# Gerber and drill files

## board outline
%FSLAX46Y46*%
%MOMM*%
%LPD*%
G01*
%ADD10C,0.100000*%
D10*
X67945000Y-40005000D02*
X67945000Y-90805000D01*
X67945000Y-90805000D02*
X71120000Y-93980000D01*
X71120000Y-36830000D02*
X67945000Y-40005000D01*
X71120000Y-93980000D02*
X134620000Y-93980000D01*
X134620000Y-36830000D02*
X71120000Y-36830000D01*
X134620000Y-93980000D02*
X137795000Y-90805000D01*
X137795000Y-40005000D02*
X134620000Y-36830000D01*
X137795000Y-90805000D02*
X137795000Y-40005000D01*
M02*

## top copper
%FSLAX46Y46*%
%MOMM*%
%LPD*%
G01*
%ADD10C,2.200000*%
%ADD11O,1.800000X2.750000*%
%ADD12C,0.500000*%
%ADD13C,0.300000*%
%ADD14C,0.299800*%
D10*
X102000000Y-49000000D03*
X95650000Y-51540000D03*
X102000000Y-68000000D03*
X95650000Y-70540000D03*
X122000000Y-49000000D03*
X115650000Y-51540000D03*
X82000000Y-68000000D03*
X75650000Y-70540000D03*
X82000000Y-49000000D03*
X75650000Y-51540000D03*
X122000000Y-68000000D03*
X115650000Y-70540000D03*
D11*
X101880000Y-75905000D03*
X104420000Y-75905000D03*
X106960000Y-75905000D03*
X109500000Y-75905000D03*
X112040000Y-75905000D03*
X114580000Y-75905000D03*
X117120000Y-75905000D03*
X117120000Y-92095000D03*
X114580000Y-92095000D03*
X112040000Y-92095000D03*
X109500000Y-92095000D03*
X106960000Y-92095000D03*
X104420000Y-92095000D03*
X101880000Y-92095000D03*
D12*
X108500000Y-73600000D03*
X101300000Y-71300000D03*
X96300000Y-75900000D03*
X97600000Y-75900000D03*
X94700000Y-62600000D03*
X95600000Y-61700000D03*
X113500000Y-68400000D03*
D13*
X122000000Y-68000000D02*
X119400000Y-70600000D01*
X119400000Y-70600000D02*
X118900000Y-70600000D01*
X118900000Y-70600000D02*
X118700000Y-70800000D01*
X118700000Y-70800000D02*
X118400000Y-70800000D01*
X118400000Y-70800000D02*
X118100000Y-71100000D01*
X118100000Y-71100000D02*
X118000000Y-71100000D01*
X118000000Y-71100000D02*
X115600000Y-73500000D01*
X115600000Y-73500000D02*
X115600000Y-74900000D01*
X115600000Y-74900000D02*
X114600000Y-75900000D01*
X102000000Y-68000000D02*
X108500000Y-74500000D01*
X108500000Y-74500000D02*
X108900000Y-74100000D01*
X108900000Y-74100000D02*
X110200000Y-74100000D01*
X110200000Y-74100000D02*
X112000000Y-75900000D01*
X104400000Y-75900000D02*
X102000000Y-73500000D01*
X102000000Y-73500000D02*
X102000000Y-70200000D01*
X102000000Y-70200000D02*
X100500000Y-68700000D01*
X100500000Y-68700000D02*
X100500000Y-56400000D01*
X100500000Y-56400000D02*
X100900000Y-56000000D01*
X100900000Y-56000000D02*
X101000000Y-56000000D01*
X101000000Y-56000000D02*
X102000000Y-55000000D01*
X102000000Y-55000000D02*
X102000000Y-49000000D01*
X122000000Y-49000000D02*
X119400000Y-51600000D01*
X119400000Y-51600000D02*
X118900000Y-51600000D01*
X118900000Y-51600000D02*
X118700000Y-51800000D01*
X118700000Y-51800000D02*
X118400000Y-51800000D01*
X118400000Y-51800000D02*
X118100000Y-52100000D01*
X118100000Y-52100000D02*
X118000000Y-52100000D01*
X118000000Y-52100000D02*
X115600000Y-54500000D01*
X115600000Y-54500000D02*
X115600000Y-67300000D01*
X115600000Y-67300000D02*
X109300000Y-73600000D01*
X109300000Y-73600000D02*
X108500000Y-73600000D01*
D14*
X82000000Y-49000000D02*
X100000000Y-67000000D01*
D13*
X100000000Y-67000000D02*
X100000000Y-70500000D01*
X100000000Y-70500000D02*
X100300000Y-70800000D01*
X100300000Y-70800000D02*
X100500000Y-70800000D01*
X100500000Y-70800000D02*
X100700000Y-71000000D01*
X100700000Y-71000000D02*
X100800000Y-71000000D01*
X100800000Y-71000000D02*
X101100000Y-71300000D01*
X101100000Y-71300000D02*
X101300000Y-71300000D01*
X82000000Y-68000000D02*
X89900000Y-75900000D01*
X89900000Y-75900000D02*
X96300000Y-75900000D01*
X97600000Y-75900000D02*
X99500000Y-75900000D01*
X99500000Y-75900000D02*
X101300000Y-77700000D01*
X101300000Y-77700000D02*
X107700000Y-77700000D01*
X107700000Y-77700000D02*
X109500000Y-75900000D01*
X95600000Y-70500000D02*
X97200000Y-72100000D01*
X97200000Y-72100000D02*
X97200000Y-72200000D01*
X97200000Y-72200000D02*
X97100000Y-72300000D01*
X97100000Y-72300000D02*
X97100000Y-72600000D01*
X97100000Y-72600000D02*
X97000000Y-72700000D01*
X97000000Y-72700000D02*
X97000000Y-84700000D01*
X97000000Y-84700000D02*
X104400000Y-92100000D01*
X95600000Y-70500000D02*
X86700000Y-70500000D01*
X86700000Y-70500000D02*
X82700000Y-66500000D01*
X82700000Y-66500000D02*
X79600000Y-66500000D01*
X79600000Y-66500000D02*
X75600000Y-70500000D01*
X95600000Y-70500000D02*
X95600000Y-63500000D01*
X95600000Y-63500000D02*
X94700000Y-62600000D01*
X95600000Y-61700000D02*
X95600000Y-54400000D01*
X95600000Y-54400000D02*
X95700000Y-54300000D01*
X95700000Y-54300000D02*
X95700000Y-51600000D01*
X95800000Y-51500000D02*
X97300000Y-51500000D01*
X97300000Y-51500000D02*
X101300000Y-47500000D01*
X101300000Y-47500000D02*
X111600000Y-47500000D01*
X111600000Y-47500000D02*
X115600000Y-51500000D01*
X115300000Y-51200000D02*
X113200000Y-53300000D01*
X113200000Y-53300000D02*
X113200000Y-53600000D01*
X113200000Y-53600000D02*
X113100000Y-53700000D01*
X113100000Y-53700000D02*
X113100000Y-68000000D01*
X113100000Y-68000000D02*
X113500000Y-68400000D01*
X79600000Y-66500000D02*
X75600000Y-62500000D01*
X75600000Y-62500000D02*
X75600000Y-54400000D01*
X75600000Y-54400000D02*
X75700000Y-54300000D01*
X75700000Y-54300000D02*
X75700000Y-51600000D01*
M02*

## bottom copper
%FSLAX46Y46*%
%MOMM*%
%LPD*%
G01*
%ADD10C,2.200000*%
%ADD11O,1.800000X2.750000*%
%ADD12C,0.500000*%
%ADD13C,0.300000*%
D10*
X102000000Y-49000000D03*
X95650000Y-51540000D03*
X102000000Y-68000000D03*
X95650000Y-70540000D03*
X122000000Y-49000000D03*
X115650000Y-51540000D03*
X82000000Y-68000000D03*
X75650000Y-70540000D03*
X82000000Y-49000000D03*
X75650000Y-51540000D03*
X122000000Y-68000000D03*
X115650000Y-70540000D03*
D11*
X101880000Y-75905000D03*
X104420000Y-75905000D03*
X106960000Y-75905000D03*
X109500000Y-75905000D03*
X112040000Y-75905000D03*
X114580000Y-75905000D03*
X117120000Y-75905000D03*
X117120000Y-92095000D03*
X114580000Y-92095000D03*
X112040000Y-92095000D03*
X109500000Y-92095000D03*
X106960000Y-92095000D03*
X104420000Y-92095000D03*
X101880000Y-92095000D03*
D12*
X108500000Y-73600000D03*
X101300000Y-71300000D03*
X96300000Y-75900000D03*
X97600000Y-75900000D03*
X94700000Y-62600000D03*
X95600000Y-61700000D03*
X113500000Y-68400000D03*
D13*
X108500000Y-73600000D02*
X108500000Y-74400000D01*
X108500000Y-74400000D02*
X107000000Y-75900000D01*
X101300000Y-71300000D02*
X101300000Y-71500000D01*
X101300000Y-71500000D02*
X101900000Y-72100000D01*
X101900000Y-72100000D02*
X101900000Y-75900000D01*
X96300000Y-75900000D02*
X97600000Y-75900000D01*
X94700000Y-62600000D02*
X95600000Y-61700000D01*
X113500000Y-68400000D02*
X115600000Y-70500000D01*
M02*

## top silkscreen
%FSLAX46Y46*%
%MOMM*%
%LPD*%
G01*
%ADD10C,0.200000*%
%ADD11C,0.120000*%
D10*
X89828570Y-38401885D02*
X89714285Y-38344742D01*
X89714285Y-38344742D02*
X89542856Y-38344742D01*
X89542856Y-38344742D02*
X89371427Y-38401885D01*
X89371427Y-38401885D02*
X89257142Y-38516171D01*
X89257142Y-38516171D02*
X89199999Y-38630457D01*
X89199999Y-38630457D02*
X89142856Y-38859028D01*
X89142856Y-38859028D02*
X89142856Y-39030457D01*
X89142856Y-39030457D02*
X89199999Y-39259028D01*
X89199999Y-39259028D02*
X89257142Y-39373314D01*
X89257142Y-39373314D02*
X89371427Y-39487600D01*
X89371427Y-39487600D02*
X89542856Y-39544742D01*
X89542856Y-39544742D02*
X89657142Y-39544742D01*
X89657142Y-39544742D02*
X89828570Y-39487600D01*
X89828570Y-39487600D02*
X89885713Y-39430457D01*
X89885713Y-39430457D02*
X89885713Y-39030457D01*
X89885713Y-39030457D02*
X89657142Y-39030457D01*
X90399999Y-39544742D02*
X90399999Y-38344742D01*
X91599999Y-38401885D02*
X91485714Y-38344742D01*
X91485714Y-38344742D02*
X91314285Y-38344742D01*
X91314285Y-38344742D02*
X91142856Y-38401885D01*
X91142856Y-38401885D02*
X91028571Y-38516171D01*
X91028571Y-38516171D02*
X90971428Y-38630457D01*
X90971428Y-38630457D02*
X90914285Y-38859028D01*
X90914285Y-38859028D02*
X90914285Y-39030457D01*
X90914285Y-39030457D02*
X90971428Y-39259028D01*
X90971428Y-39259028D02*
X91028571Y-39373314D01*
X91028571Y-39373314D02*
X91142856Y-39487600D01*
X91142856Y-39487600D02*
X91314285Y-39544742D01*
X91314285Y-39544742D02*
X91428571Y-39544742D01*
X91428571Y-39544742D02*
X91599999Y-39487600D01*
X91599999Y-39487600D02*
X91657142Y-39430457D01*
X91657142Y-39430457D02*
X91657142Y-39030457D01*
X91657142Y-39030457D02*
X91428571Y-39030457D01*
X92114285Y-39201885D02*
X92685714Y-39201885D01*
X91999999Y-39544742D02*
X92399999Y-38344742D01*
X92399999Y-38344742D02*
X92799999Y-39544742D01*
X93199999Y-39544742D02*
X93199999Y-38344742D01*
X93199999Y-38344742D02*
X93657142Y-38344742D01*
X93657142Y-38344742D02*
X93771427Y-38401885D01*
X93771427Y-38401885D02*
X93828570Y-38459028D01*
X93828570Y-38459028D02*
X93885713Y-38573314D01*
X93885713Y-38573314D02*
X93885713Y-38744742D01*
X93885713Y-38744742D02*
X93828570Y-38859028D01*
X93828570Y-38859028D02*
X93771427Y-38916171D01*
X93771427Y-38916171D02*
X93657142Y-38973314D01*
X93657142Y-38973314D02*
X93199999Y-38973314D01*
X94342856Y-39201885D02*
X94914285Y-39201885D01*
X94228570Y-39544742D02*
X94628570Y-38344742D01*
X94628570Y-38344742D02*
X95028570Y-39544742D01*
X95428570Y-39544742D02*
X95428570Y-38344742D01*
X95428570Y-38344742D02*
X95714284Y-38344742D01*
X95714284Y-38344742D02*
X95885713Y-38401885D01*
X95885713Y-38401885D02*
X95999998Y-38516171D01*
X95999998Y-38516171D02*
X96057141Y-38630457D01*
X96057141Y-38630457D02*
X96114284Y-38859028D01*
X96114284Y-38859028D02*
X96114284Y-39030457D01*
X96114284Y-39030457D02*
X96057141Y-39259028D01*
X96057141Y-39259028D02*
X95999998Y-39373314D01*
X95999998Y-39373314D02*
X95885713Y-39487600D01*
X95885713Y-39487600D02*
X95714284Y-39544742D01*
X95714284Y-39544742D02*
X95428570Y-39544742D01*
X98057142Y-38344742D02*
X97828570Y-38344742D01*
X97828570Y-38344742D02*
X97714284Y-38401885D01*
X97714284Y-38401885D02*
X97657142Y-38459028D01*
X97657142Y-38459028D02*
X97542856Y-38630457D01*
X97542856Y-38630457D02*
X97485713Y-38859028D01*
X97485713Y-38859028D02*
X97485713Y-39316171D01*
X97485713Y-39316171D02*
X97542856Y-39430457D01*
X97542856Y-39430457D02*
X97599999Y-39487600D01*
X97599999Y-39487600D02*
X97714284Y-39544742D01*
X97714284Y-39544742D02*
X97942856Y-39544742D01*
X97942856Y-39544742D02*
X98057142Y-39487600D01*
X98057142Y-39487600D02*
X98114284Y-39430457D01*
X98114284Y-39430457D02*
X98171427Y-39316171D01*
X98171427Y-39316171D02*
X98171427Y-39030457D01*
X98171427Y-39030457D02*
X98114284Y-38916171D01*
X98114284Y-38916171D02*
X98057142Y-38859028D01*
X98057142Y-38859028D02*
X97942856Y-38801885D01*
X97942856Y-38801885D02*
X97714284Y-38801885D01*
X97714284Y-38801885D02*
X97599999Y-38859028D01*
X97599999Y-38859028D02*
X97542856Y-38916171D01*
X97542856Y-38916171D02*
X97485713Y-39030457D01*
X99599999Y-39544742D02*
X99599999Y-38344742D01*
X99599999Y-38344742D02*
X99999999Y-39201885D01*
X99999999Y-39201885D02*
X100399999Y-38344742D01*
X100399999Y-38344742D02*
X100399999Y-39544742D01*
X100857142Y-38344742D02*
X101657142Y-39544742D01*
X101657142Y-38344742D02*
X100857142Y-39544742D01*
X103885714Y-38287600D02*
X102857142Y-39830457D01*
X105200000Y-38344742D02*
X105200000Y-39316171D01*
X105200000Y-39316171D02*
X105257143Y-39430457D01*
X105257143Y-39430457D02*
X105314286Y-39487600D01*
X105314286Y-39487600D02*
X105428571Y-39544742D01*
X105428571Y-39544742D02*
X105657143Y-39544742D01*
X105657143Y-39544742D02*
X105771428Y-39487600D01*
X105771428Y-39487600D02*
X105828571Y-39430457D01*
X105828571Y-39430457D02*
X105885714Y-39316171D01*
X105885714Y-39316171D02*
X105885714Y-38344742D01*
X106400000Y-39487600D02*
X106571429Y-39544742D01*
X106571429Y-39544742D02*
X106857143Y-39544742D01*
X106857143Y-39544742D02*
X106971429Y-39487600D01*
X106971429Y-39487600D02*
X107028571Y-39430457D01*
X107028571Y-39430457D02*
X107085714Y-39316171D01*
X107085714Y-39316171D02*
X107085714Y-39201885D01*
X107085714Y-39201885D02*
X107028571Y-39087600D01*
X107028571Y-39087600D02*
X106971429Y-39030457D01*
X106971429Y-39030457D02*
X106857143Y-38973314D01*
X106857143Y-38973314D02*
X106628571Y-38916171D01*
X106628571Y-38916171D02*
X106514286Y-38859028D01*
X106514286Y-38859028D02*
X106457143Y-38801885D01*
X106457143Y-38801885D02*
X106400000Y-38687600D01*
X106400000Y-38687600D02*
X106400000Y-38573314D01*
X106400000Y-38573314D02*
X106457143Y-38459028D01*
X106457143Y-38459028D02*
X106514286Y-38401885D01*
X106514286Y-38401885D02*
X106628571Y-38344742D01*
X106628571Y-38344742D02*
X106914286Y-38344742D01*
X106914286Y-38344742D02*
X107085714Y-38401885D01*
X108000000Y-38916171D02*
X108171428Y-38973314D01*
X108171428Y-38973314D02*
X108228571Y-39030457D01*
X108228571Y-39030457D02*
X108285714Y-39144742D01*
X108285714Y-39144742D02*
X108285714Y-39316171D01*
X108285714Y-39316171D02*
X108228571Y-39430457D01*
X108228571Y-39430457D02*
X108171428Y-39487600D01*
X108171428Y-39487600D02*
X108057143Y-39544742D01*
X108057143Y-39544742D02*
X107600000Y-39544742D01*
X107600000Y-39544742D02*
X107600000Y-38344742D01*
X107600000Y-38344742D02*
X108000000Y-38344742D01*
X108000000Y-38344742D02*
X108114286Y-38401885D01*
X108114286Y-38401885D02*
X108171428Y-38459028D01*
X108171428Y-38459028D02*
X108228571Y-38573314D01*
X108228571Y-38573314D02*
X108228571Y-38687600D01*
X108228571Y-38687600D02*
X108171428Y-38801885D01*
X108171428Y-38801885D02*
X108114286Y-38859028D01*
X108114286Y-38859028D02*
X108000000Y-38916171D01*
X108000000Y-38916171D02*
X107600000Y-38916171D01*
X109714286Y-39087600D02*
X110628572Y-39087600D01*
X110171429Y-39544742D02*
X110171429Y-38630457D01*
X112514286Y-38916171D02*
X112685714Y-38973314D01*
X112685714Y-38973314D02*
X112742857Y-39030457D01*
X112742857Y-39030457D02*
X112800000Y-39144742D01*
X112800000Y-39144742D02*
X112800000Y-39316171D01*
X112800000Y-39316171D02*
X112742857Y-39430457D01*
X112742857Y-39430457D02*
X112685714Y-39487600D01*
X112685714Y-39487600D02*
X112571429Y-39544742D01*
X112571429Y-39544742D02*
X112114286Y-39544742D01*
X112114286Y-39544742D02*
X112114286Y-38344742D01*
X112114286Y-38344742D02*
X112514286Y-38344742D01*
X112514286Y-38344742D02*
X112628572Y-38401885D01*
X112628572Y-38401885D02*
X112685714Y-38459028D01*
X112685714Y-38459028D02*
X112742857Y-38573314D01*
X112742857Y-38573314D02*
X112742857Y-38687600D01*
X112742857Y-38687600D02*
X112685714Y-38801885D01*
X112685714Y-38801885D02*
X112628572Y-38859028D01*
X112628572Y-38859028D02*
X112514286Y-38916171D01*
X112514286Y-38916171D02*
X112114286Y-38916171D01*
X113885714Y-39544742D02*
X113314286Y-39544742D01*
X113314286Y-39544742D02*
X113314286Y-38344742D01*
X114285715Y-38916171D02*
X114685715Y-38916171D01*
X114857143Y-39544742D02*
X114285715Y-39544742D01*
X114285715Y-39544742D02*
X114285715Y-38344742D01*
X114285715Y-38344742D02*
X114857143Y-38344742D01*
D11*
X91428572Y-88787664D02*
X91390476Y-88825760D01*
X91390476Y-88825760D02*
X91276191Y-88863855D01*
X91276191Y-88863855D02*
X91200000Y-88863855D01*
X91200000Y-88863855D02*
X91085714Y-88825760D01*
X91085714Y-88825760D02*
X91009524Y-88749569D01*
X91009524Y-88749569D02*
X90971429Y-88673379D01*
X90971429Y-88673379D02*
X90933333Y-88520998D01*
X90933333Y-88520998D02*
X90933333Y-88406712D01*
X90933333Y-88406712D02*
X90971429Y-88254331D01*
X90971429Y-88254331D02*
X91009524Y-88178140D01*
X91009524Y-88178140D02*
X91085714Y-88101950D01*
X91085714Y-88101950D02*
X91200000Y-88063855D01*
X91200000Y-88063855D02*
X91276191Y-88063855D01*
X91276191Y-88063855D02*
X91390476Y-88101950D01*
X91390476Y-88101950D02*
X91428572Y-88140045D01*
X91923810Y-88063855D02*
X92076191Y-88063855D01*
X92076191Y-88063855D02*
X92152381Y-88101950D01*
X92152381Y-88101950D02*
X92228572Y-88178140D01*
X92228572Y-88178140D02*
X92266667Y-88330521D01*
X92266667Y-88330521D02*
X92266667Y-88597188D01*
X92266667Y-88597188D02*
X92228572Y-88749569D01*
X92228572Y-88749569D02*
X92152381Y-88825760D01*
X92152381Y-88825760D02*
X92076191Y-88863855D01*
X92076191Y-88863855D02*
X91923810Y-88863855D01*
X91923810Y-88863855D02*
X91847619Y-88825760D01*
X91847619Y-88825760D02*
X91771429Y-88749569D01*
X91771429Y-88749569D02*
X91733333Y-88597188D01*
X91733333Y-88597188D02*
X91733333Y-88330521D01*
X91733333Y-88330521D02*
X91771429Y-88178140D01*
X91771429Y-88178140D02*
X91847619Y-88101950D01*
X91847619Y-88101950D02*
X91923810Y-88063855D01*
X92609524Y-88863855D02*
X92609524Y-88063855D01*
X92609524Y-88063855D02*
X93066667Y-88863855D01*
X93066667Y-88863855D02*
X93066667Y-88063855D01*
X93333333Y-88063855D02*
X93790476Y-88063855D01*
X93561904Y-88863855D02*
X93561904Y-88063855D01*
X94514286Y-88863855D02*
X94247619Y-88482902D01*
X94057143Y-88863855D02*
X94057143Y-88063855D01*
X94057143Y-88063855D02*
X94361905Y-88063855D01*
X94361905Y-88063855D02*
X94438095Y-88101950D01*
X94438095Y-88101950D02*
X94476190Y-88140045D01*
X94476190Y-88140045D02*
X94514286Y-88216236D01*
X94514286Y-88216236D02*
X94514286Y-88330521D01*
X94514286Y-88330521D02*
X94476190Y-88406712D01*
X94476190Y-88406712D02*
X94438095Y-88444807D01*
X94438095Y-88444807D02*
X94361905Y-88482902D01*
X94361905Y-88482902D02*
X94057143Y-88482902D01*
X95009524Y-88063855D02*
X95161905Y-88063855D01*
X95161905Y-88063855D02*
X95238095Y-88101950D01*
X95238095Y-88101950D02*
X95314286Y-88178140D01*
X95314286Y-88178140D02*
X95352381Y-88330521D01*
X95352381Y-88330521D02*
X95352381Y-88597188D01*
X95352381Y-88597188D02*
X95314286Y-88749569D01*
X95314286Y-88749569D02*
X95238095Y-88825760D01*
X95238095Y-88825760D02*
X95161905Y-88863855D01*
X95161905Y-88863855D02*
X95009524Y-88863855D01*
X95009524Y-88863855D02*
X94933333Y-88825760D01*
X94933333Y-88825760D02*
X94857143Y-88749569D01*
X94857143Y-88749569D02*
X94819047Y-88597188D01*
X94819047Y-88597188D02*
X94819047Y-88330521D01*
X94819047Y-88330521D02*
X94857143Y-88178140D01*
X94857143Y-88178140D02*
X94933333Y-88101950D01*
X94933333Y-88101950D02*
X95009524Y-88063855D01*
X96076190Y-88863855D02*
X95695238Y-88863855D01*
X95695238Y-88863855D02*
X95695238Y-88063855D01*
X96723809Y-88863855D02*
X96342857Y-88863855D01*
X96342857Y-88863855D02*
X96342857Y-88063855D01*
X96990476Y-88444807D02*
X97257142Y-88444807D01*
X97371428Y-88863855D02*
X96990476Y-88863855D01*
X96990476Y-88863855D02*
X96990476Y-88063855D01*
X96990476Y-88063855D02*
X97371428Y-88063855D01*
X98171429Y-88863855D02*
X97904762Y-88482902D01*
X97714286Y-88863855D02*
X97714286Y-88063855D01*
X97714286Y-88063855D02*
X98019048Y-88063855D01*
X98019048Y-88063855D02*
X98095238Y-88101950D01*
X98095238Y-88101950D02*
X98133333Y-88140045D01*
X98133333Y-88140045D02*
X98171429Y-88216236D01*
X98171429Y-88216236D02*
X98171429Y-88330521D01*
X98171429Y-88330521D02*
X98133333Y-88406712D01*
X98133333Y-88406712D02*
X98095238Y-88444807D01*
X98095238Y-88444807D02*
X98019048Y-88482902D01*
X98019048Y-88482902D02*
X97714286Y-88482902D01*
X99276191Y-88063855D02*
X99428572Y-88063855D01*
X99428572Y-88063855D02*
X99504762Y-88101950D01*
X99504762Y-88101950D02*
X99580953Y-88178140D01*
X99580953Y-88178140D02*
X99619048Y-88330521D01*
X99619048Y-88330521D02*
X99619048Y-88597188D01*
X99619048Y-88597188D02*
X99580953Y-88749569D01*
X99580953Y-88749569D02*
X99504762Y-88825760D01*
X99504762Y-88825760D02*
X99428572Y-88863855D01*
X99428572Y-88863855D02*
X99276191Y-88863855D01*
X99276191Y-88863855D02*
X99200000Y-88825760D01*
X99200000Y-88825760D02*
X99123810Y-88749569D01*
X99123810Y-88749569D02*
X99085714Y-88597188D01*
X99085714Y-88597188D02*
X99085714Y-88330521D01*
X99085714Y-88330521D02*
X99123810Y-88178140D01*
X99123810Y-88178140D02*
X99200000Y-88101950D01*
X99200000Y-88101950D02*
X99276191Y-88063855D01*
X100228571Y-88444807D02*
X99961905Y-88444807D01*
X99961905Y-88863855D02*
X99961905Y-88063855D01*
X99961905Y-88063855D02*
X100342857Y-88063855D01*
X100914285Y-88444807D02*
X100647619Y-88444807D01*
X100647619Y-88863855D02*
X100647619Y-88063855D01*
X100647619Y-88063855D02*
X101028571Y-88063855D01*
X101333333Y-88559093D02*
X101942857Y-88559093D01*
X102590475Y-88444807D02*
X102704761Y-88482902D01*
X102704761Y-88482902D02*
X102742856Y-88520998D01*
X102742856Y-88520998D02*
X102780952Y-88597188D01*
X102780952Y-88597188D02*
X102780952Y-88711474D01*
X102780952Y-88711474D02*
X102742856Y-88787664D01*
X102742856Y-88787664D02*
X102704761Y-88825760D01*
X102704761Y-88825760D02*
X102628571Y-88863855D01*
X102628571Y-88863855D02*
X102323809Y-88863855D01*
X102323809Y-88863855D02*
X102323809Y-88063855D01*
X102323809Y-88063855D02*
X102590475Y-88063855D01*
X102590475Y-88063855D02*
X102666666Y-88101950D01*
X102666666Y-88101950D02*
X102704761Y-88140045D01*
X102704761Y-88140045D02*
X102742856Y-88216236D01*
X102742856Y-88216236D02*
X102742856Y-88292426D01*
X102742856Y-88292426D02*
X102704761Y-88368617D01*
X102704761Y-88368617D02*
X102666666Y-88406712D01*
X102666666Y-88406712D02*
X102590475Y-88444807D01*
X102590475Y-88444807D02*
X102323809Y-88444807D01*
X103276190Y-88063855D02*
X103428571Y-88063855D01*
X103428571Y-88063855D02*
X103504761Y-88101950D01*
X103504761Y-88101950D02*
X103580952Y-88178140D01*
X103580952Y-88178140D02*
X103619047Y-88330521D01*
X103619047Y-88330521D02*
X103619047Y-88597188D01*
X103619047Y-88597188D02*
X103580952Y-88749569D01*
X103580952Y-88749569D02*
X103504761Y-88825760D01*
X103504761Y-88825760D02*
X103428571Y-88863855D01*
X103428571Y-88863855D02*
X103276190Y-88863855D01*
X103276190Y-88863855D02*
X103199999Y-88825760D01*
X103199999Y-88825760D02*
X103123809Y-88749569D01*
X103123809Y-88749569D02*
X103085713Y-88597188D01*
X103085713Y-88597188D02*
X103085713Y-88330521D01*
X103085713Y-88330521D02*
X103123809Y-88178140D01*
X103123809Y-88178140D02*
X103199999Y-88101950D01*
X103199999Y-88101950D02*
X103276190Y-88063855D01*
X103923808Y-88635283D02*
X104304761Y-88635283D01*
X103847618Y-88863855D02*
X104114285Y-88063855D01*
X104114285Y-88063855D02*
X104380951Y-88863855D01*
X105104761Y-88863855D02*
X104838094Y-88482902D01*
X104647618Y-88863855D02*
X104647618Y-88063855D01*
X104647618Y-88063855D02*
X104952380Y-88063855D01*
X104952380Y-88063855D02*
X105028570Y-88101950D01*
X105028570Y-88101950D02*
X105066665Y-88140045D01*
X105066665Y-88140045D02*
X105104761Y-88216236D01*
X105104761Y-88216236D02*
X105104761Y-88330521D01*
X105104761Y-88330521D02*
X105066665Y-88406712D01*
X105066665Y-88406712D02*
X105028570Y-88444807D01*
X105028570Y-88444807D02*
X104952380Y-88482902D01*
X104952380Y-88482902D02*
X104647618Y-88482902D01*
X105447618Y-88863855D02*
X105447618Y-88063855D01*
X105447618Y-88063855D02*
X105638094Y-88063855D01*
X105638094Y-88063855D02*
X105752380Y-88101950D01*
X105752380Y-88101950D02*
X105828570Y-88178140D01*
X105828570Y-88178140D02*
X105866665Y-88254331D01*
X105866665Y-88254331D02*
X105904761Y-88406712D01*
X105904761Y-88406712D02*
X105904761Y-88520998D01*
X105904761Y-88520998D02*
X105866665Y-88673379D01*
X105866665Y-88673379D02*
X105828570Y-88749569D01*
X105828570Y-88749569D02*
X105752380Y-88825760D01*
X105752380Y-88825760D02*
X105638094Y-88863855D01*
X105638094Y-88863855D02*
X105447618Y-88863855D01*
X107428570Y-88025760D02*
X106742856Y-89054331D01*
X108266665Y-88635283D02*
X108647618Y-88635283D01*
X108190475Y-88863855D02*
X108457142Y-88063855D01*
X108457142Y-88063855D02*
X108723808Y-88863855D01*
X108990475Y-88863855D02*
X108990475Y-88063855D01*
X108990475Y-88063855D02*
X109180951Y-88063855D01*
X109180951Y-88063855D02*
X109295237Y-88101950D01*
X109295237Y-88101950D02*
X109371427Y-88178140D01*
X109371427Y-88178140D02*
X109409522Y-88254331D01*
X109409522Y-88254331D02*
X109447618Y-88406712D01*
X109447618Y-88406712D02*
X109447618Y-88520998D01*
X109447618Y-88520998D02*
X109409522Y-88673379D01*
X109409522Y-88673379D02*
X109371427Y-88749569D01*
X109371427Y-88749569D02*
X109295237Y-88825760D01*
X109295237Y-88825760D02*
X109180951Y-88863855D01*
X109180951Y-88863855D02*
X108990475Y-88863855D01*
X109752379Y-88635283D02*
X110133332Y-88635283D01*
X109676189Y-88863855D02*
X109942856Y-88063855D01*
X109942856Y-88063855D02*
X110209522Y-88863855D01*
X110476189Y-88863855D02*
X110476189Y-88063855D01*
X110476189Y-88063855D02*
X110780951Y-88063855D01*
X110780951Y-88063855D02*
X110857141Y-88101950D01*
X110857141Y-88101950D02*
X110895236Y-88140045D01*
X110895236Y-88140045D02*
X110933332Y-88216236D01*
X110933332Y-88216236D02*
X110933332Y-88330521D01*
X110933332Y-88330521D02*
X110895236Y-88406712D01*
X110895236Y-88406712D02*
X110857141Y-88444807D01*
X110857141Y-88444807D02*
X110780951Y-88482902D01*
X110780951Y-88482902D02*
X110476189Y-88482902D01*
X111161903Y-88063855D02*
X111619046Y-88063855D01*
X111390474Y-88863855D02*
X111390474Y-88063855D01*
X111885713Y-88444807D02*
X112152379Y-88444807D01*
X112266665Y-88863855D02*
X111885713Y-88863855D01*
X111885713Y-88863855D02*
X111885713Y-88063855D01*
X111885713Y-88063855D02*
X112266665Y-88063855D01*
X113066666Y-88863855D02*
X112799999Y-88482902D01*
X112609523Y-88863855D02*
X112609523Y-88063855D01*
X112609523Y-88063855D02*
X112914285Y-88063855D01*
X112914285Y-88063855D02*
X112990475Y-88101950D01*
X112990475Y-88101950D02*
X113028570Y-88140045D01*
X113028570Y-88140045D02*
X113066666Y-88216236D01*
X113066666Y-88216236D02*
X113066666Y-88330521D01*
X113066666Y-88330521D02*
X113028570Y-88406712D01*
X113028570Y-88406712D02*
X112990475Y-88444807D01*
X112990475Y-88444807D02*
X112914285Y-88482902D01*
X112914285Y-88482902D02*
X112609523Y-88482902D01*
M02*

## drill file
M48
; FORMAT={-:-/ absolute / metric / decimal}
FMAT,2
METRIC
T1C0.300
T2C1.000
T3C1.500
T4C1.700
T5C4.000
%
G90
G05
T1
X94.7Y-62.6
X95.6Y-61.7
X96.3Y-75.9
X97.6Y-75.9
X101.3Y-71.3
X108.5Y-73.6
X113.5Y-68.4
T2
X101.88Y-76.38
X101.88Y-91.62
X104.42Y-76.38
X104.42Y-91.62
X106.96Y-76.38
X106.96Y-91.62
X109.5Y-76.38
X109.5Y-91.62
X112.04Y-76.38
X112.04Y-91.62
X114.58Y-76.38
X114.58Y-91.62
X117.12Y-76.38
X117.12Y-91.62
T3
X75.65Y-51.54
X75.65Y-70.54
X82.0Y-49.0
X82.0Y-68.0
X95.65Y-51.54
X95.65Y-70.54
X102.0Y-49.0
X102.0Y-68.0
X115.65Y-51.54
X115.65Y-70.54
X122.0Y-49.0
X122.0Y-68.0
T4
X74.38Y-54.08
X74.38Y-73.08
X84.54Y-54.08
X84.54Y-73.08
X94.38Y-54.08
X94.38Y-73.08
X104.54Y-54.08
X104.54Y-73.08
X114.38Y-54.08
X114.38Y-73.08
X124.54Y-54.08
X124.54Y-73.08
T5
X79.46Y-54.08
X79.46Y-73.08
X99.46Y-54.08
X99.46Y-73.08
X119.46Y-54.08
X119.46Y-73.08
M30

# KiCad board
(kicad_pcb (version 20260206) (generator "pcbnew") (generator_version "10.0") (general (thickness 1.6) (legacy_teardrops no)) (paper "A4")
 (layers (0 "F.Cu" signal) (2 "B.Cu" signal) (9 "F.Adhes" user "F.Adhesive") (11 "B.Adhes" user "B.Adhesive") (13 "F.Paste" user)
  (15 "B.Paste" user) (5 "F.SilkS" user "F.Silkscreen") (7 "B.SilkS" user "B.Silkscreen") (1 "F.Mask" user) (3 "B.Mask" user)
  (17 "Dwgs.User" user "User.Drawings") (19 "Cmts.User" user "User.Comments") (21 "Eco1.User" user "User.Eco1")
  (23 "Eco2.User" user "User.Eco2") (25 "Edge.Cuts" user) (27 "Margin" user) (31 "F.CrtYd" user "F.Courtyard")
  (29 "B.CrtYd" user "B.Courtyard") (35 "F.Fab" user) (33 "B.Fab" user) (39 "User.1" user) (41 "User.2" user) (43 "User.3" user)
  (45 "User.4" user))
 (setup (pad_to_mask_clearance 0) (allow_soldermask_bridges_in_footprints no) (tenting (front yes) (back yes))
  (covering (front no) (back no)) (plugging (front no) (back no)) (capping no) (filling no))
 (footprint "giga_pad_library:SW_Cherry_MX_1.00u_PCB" (layer "F.Cu") (at 102 49)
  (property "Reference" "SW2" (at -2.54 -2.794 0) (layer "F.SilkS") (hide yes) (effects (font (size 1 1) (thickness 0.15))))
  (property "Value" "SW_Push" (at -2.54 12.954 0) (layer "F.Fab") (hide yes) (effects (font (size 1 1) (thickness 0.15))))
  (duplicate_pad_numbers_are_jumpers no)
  (pad "" np_thru_hole circle (at -7.62 5.08) (size 1.7 1.7) (drill 1.7) (layers "*.Cu" "*.Mask"))
  (pad "" np_thru_hole circle (at -2.54 5.08) (size 4 4) (drill 4) (layers "*.Cu" "*.Mask"))
  (pad "" np_thru_hole circle (at 2.54 5.08) (size 1.7 1.7) (drill 1.7) (layers "*.Cu" "*.Mask"))
  (pad "1" thru_hole circle (at 0 0) (size 2.2 2.2) (drill 1.5) (layers "*.Cu" "*.Mask") (remove_unused_layers no) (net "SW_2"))
  (pad "2" thru_hole circle (at -6.35 2.54) (size 2.2 2.2) (drill 1.5) (layers "*.Cu" "*.Mask") (remove_unused_layers no) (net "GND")))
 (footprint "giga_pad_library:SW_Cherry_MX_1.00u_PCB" (layer "F.Cu") (at 102 68)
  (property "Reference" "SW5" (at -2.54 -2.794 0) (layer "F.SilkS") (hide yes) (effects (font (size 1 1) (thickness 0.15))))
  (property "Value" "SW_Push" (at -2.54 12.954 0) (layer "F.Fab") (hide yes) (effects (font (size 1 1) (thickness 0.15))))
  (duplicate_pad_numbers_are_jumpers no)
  (pad "" np_thru_hole circle (at -7.62 5.08) (size 1.7 1.7) (drill 1.7) (layers "*.Cu" "*.Mask"))
  (pad "" np_thru_hole circle (at -2.54 5.08) (size 4 4) (drill 4) (layers "*.Cu" "*.Mask"))
  (pad "" np_thru_hole circle (at 2.54 5.08) (size 1.7 1.7) (drill 1.7) (layers "*.Cu" "*.Mask"))
  (pad "1" thru_hole circle (at 0 0) (size 2.2 2.2) (drill 1.5) (layers "*.Cu" "*.Mask") (remove_unused_layers no) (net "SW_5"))
  (pad "2" thru_hole circle (at -6.35 2.54) (size 2.2 2.2) (drill 1.5) (layers "*.Cu" "*.Mask") (remove_unused_layers no) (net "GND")))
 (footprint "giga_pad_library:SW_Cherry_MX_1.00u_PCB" (layer "F.Cu") (at 122 49)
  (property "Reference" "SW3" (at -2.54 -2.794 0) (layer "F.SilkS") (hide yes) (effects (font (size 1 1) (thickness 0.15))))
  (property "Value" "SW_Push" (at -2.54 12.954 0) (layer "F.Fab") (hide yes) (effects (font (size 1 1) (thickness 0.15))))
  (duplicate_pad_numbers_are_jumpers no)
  (pad "" np_thru_hole circle (at -7.62 5.08) (size 1.7 1.7) (drill 1.7) (layers "*.Cu" "*.Mask"))
  (pad "" np_thru_hole circle (at -2.54 5.08) (size 4 4) (drill 4) (layers "*.Cu" "*.Mask"))
  (pad "" np_thru_hole circle (at 2.54 5.08) (size 1.7 1.7) (drill 1.7) (layers "*.Cu" "*.Mask"))
  (pad "1" thru_hole circle (at 0 0) (size 2.2 2.2) (drill 1.5) (layers "*.Cu" "*.Mask") (remove_unused_layers no) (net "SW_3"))
  (pad "2" thru_hole circle (at -6.35 2.54) (size 2.2 2.2) (drill 1.5) (layers "*.Cu" "*.Mask") (remove_unused_layers no) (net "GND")))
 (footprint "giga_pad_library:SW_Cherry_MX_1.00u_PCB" (layer "F.Cu") (at 82 68)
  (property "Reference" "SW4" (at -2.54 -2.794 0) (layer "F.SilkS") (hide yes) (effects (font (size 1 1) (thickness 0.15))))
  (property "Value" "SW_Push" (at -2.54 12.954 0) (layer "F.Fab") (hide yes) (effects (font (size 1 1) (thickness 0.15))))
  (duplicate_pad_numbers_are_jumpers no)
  (pad "" np_thru_hole circle (at -7.62 5.08) (size 1.7 1.7) (drill 1.7) (layers "*.Cu" "*.Mask"))
  (pad "" np_thru_hole circle (at -2.54 5.08) (size 4 4) (drill 4) (layers "*.Cu" "*.Mask"))
  (pad "" np_thru_hole circle (at 2.54 5.08) (size 1.7 1.7) (drill 1.7) (layers "*.Cu" "*.Mask"))
  (pad "1" thru_hole circle (at 0 0) (size 2.2 2.2) (drill 1.5) (layers "*.Cu" "*.Mask") (remove_unused_layers no) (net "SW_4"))
  (pad "2" thru_hole circle (at -6.35 2.54) (size 2.2 2.2) (drill 1.5) (layers "*.Cu" "*.Mask") (remove_unused_layers no) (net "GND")))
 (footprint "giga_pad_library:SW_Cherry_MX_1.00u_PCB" (layer "F.Cu") (at 82 49)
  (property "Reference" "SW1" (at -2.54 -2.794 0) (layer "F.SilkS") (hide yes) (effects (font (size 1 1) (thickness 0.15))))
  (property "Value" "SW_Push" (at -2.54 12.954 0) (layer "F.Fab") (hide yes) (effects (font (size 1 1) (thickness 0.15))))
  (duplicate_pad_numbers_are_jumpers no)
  (pad "" np_thru_hole circle (at -7.62 5.08) (size 1.7 1.7) (drill 1.7) (layers "*.Cu" "*.Mask"))
  (pad "" np_thru_hole circle (at -2.54 5.08) (size 4 4) (drill 4) (layers "*.Cu" "*.Mask"))
  (pad "" np_thru_hole circle (at 2.54 5.08) (size 1.7 1.7) (drill 1.7) (layers "*.Cu" "*.Mask"))
  (pad "1" thru_hole circle (at 0 0) (size 2.2 2.2) (drill 1.5) (layers "*.Cu" "*.Mask") (remove_unused_layers no) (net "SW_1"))
  (pad "2" thru_hole circle (at -6.35 2.54) (size 2.2 2.2) (drill 1.5) (layers "*.Cu" "*.Mask") (remove_unused_layers no) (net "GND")))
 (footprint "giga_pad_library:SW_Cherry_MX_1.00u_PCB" (layer "F.Cu") (at 122 68)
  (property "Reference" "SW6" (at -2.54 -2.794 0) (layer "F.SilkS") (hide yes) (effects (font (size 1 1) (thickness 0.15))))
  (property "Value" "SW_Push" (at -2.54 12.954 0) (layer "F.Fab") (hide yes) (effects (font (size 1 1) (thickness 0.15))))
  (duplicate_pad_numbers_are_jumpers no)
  (pad "" np_thru_hole circle (at -7.62 5.08) (size 1.7 1.7) (drill 1.7) (layers "*.Cu" "*.Mask"))
  (pad "" np_thru_hole circle (at -2.54 5.08) (size 4 4) (drill 4) (layers "*.Cu" "*.Mask"))
  (pad "" np_thru_hole circle (at 2.54 5.08) (size 1.7 1.7) (drill 1.7) (layers "*.Cu" "*.Mask"))
  (pad "1" thru_hole circle (at 0 0) (size 2.2 2.2) (drill 1.5) (layers "*.Cu" "*.Mask") (remove_unused_layers no) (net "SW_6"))
  (pad "2" thru_hole circle (at -6.35 2.54) (size 2.2 2.2) (drill 1.5) (layers "*.Cu" "*.Mask") (remove_unused_layers no) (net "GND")))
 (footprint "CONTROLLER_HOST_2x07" (layer "B.Cu") (at 109.5000 84 -90)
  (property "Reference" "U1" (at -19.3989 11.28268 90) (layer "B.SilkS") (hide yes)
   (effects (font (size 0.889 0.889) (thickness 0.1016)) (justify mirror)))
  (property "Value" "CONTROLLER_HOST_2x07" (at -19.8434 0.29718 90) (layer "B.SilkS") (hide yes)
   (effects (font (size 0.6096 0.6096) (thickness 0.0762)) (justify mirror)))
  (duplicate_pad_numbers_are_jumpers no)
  (pad "1" thru_hole oval (at -7.62 7.62 270) (size 2.75 1.8) (drill 1 (offset -0.475 0)) (layers "*.Cu" "*.Mask") (remove_unused_layers no)
   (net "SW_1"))
  (pad "2" thru_hole oval (at -7.62 5.08 270) (size 2.75 1.8) (drill 1 (offset -0.475 0)) (layers "*.Cu" "*.Mask") (remove_unused_layers no)
   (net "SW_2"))
  (pad "3" thru_hole oval (at -7.62 2.54 270) (size 2.75 1.8) (drill 1 (offset -0.475 0)) (layers "*.Cu" "*.Mask") (remove_unused_layers no)
   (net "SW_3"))
  (pad "4" thru_hole oval (at -7.62 0 270) (size 2.75 1.8) (drill 1 (offset -0.475 0)) (layers "*.Cu" "*.Mask") (remove_unused_layers no)
   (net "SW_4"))
  (pad "5" thru_hole oval (at -7.62 -2.54 270) (size 2.75 1.8) (drill 1 (offset -0.475 0)) (layers "*.Cu" "*.Mask")
   (remove_unused_layers no) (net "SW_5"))
  (pad "6" thru_hole oval (at -7.62 -5.08 270) (size 2.75 1.8) (drill 1 (offset -0.475 0)) (layers "*.Cu" "*.Mask")
   (remove_unused_layers no) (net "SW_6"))
  (pad "7" thru_hole oval (at -7.62 -7.62 270) (size 2.75 1.8) (drill 1 (offset -0.475 0)) (layers "*.Cu" "*.Mask")
   (remove_unused_layers no))
  (pad "8" thru_hole oval (at 7.62 -7.62 90) (size 2.75 1.8) (drill 1 (offset -0.475 0)) (layers "*.Cu" "*.Mask") (remove_unused_layers no))
  (pad "9" thru_hole oval (at 7.62 -5.08 90) (size 2.75 1.8) (drill 1 (offset -0.475 0)) (layers "*.Cu" "*.Mask") (remove_unused_layers no))
  (pad "10" thru_hole oval (at 7.62 -2.54 90) (size 2.75 1.8) (drill 1 (offset -0.475 0)) (layers "*.Cu" "*.Mask") (remove_unused_layers no))
  (pad "11" thru_hole oval (at 7.62 0 90) (size 2.75 1.8) (drill 1 (offset -0.475 0)) (layers "*.Cu" "*.Mask") (remove_unused_layers no))
  (pad "12" thru_hole oval (at 7.62 2.54 90) (size 2.75 1.8) (drill 1 (offset -0.475 0)) (layers "*.Cu" "*.Mask") (remove_unused_layers no))
  (pad "13" thru_hole oval (at 7.62 5.08 90) (size 2.75 1.8) (drill 1 (offset -0.475 0)) (layers "*.Cu" "*.Mask") (remove_unused_layers no)
   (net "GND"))
  (pad "14" thru_hole oval (at 7.62 7.62 90) (size 2.75 1.8) (drill 1 (offset -0.475 0)) (layers "*.Cu" "*.Mask") (remove_unused_layers no)))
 (gr_line (start 67.945 40.005) (end 67.945 90.805) (stroke (width 0.1) (type default)) (layer "Edge.Cuts"))
 (gr_line (start 67.945 90.805) (end 71.12 93.98) (stroke (width 0.1) (type default)) (layer "Edge.Cuts"))
 (gr_line (start 71.12 36.83) (end 67.945 40.005) (stroke (width 0.1) (type default)) (layer "Edge.Cuts"))
 (gr_line (start 71.12 93.98) (end 134.62 93.98) (stroke (width 0.1) (type default)) (layer "Edge.Cuts"))
 (gr_line (start 134.62 36.83) (end 71.12 36.83) (stroke (width 0.1) (type default)) (layer "Edge.Cuts"))
 (gr_line (start 134.62 93.98) (end 137.795 90.805) (stroke (width 0.1) (type default)) (layer "Edge.Cuts"))
 (gr_line (start 137.795 40.005) (end 134.62 36.83) (stroke (width 0.1) (type default)) (layer "Edge.Cuts"))
 (gr_line (start 137.795 90.805) (end 137.795 40.005) (stroke (width 0.1) (type default)) (layer "Edge.Cuts"))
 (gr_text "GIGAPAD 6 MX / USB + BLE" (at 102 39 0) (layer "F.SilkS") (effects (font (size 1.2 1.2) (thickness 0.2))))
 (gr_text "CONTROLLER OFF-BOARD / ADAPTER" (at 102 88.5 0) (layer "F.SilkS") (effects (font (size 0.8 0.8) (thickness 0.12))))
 (segment (start 122.000000 68.000000) (end 119.400000 70.600000) (width 0.3) (layer "F.Cu") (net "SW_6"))
 (segment (start 119.400000 70.600000) (end 118.900000 70.600000) (width 0.3) (layer "F.Cu") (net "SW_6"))
 (segment (start 118.900000 70.600000) (end 118.700000 70.800000) (width 0.3) (layer "F.Cu") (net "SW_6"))
 (segment (start 118.700000 70.800000) (end 118.400000 70.800000) (width 0.3) (layer "F.Cu") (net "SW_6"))
 (segment (start 118.400000 70.800000) (end 118.100000 71.100000) (width 0.3) (layer "F.Cu") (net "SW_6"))
 (segment (start 118.100000 71.100000) (end 118.000000 71.100000) (width 0.3) (layer "F.Cu") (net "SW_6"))
 (segment (start 118.000000 71.100000) (end 115.600000 73.500000) (width 0.3) (layer "F.Cu") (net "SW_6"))
 (segment (start 115.600000 73.500000) (end 115.600000 74.900000) (width 0.3) (layer "F.Cu") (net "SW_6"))
 (segment (start 115.600000 74.900000) (end 114.600000 75.900000) (width 0.3) (layer "F.Cu") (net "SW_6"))
 (segment (start 102.000000 68.000000) (end 108.500000 74.500000) (width 0.3) (layer "F.Cu") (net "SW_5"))
 (segment (start 108.500000 74.500000) (end 108.900000 74.100000) (width 0.3) (layer "F.Cu") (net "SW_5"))
 (segment (start 108.900000 74.100000) (end 110.200000 74.100000) (width 0.3) (layer "F.Cu") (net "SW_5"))
 (segment (start 110.200000 74.100000) (end 112.000000 75.900000) (width 0.3) (layer "F.Cu") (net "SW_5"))
 (segment (start 104.400000 75.900000) (end 102.000000 73.500000) (width 0.3) (layer "F.Cu") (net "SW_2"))
 (segment (start 102.000000 73.500000) (end 102.000000 70.200000) (width 0.3) (layer "F.Cu") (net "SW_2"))
 (segment (start 102.000000 70.200000) (end 100.500000 68.700000) (width 0.3) (layer "F.Cu") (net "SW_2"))
 (segment (start 100.500000 68.700000) (end 100.500000 56.400000) (width 0.3) (layer "F.Cu") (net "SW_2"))
 (segment (start 100.500000 56.400000) (end 100.900000 56.000000) (width 0.3) (layer "F.Cu") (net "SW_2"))
 (segment (start 100.900000 56.000000) (end 101.000000 56.000000) (width 0.3) (layer "F.Cu") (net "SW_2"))
 (segment (start 101.000000 56.000000) (end 102.000000 55.000000) (width 0.3) (layer "F.Cu") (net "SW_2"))
 (segment (start 102.000000 55.000000) (end 102.000000 49.000000) (width 0.3) (layer "F.Cu") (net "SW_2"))
 (segment (start 122.000000 49.000000) (end 119.400000 51.600000) (width 0.3) (layer "F.Cu") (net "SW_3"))
 (segment (start 119.400000 51.600000) (end 118.900000 51.600000) (width 0.3) (layer "F.Cu") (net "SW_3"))
 (segment (start 118.900000 51.600000) (end 118.700000 51.800000) (width 0.3) (layer "F.Cu") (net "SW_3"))
 (segment (start 118.700000 51.800000) (end 118.400000 51.800000) (width 0.3) (layer "F.Cu") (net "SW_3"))
 (segment (start 118.400000 51.800000) (end 118.100000 52.100000) (width 0.3) (layer "F.Cu") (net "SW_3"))
 (segment (start 118.100000 52.100000) (end 118.000000 52.100000) (width 0.3) (layer "F.Cu") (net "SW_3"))
 (segment (start 118.000000 52.100000) (end 115.600000 54.500000) (width 0.3) (layer "F.Cu") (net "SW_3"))
 (segment (start 115.600000 54.500000) (end 115.600000 67.300000) (width 0.3) (layer "F.Cu") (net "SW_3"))
 (segment (start 115.600000 67.300000) (end 109.300000 73.600000) (width 0.3) (layer "F.Cu") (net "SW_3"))
 (segment (start 109.300000 73.600000) (end 108.500000 73.600000) (width 0.3) (layer "F.Cu") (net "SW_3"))
 (segment (start 108.500000 73.600000) (end 108.500000 74.400000) (width 0.3) (layer "B.Cu") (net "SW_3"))
 (segment (start 108.500000 74.400000) (end 107.000000 75.900000) (width 0.3) (layer "B.Cu") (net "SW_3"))
 (via (at 108.500000 73.600000) (size 0.5) (drill 0.3) (layers "F.Cu" "B.Cu") (tenting (front yes) (back yes)) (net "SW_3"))
 (segment (start 82.000000 49.000000) (end 100.000000 67.000000) (width 0.2998) (layer "F.Cu") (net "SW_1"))
 (segment (start 100.000000 67.000000) (end 100.000000 70.500000) (width 0.3) (layer "F.Cu") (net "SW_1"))
 (segment (start 100.000000 70.500000) (end 100.300000 70.800000) (width 0.3) (layer "F.Cu") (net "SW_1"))
 (segment (start 100.300000 70.800000) (end 100.500000 70.800000) (width 0.3) (layer "F.Cu") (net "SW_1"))
 (segment (start 100.500000 70.800000) (end 100.700000 71.000000) (width 0.3) (layer "F.Cu") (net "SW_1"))
 (segment (start 100.700000 71.000000) (end 100.800000 71.000000) (width 0.3) (layer "F.Cu") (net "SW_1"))
 (segment (start 100.800000 71.000000) (end 101.100000 71.300000) (width 0.3) (layer "F.Cu") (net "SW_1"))
 (segment (start 101.100000 71.300000) (end 101.300000 71.300000) (width 0.3) (layer "F.Cu") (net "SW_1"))
 (segment (start 101.300000 71.300000) (end 101.300000 71.500000) (width 0.3) (layer "B.Cu") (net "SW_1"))
 (segment (start 101.300000 71.500000) (end 101.900000 72.100000) (width 0.3) (layer "B.Cu") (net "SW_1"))
 (segment (start 101.900000 72.100000) (end 101.900000 75.900000) (width 0.3) (layer "B.Cu") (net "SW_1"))
 (via (at 101.300000 71.300000) (size 0.5) (drill 0.3) (layers "F.Cu" "B.Cu") (tenting (front yes) (back yes)) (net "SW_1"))
 (segment (start 82.000000 68.000000) (end 89.900000 75.900000) (width 0.3) (layer "F.Cu") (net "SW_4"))
 (segment (start 89.900000 75.900000) (end 96.300000 75.900000) (width 0.3) (layer "F.Cu") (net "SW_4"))
 (segment (start 96.300000 75.900000) (end 97.600000 75.900000) (width 0.3) (layer "B.Cu") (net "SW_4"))
 (segment (start 97.600000 75.900000) (end 99.500000 75.900000) (width 0.3) (layer "F.Cu") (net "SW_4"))
 (segment (start 99.500000 75.900000) (end 101.300000 77.700000) (width 0.3) (layer "F.Cu") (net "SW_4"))
 (segment (start 101.300000 77.700000) (end 107.700000 77.700000) (width 0.3) (layer "F.Cu") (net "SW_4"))
 (segment (start 107.700000 77.700000) (end 109.500000 75.900000) (width 0.3) (layer "F.Cu") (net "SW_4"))
 (via (at 96.300000 75.900000) (size 0.5) (drill 0.3) (layers "F.Cu" "B.Cu") (tenting (front yes) (back yes)) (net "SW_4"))
 (via (at 97.600000 75.900000) (size 0.5) (drill 0.3) (layers "F.Cu" "B.Cu") (tenting (front yes) (back yes)) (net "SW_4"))
 (segment (start 95.600000 70.500000) (end 97.200000 72.100000) (width 0.3) (layer "F.Cu") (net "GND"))
 (segment (start 97.200000 72.100000) (end 97.200000 72.200000) (width 0.3) (layer "F.Cu") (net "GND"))
 (segment (start 97.200000 72.200000) (end 97.100000 72.300000) (width 0.3) (layer "F.Cu") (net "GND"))
 (segment (start 97.100000 72.300000) (end 97.100000 72.600000) (width 0.3) (layer "F.Cu") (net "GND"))
 (segment (start 97.100000 72.600000) (end 97.000000 72.700000) (width 0.3) (layer "F.Cu") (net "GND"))
 (segment (start 97.000000 72.700000) (end 97.000000 84.700000) (width 0.3) (layer "F.Cu") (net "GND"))
 (segment (start 97.000000 84.700000) (end 104.400000 92.100000) (width 0.3) (layer "F.Cu") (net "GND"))
 (segment (start 95.600000 70.500000) (end 86.700000 70.500000) (width 0.3) (layer "F.Cu") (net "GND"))
 (segment (start 86.700000 70.500000) (end 82.700000 66.500000) (width 0.3) (layer "F.Cu") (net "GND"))
 (segment (start 82.700000 66.500000) (end 79.600000 66.500000) (width 0.3) (layer "F.Cu") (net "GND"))
 (segment (start 79.600000 66.500000) (end 75.600000 70.500000) (width 0.3) (layer "F.Cu") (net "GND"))
 (segment (start 95.600000 70.500000) (end 95.600000 63.500000) (width 0.3) (layer "F.Cu") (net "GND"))
 (segment (start 95.600000 63.500000) (end 94.700000 62.600000) (width 0.3) (layer "F.Cu") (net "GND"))
 (segment (start 94.700000 62.600000) (end 95.600000 61.700000) (width 0.3) (layer "B.Cu") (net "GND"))
 (segment (start 95.600000 61.700000) (end 95.600000 54.400000) (width 0.3) (layer "F.Cu") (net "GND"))
 (segment (start 95.600000 54.400000) (end 95.700000 54.300000) (width 0.3) (layer "F.Cu") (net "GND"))
 (segment (start 95.700000 54.300000) (end 95.700000 51.600000) (width 0.3) (layer "F.Cu") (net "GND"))
 (segment (start 95.800000 51.500000) (end 97.300000 51.500000) (width 0.3) (layer "F.Cu") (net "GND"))
 (segment (start 97.300000 51.500000) (end 101.300000 47.500000) (width 0.3) (layer "F.Cu") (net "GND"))
 (segment (start 101.300000 47.500000) (end 111.600000 47.500000) (width 0.3) (layer "F.Cu") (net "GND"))
 (segment (start 111.600000 47.500000) (end 115.600000 51.500000) (width 0.3) (layer "F.Cu") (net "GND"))
 (segment (start 115.300000 51.200000) (end 113.200000 53.300000) (width 0.3) (layer "F.Cu") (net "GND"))
 (segment (start 113.200000 53.300000) (end 113.200000 53.600000) (width 0.3) (layer "F.Cu") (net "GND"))
 (segment (start 113.200000 53.600000) (end 113.100000 53.700000) (width 0.3) (layer "F.Cu") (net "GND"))
 (segment (start 113.100000 53.700000) (end 113.100000 68.000000) (width 0.3) (layer "F.Cu") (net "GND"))
 (segment (start 113.100000 68.000000) (end 113.500000 68.400000) (width 0.3) (layer "F.Cu") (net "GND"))
 (segment (start 113.500000 68.400000) (end 115.600000 70.500000) (width 0.3) (layer "B.Cu") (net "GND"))
 (segment (start 79.600000 66.500000) (end 75.600000 62.500000) (width 0.3) (layer "F.Cu") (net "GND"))
 (segment (start 75.600000 62.500000) (end 75.600000 54.400000) (width 0.3) (layer "F.Cu") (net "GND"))
 (segment (start 75.600000 54.400000) (end 75.700000 54.300000) (width 0.3) (layer "F.Cu") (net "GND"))
 (segment (start 75.700000 54.300000) (end 75.700000 51.600000) (width 0.3) (layer "F.Cu") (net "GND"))
 (via (at 94.700000 62.600000) (size 0.5) (drill 0.3) (layers "F.Cu" "B.Cu") (tenting (front yes) (back yes)) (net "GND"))
 (via (at 95.600000 61.700000) (size 0.5) (drill 0.3) (layers "F.Cu" "B.Cu") (tenting (front yes) (back yes)) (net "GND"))
 (via (at 113.500000 68.400000) (size 0.5) (drill 0.3) (layers "F.Cu" "B.Cu") (tenting (front yes) (back yes)) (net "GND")))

